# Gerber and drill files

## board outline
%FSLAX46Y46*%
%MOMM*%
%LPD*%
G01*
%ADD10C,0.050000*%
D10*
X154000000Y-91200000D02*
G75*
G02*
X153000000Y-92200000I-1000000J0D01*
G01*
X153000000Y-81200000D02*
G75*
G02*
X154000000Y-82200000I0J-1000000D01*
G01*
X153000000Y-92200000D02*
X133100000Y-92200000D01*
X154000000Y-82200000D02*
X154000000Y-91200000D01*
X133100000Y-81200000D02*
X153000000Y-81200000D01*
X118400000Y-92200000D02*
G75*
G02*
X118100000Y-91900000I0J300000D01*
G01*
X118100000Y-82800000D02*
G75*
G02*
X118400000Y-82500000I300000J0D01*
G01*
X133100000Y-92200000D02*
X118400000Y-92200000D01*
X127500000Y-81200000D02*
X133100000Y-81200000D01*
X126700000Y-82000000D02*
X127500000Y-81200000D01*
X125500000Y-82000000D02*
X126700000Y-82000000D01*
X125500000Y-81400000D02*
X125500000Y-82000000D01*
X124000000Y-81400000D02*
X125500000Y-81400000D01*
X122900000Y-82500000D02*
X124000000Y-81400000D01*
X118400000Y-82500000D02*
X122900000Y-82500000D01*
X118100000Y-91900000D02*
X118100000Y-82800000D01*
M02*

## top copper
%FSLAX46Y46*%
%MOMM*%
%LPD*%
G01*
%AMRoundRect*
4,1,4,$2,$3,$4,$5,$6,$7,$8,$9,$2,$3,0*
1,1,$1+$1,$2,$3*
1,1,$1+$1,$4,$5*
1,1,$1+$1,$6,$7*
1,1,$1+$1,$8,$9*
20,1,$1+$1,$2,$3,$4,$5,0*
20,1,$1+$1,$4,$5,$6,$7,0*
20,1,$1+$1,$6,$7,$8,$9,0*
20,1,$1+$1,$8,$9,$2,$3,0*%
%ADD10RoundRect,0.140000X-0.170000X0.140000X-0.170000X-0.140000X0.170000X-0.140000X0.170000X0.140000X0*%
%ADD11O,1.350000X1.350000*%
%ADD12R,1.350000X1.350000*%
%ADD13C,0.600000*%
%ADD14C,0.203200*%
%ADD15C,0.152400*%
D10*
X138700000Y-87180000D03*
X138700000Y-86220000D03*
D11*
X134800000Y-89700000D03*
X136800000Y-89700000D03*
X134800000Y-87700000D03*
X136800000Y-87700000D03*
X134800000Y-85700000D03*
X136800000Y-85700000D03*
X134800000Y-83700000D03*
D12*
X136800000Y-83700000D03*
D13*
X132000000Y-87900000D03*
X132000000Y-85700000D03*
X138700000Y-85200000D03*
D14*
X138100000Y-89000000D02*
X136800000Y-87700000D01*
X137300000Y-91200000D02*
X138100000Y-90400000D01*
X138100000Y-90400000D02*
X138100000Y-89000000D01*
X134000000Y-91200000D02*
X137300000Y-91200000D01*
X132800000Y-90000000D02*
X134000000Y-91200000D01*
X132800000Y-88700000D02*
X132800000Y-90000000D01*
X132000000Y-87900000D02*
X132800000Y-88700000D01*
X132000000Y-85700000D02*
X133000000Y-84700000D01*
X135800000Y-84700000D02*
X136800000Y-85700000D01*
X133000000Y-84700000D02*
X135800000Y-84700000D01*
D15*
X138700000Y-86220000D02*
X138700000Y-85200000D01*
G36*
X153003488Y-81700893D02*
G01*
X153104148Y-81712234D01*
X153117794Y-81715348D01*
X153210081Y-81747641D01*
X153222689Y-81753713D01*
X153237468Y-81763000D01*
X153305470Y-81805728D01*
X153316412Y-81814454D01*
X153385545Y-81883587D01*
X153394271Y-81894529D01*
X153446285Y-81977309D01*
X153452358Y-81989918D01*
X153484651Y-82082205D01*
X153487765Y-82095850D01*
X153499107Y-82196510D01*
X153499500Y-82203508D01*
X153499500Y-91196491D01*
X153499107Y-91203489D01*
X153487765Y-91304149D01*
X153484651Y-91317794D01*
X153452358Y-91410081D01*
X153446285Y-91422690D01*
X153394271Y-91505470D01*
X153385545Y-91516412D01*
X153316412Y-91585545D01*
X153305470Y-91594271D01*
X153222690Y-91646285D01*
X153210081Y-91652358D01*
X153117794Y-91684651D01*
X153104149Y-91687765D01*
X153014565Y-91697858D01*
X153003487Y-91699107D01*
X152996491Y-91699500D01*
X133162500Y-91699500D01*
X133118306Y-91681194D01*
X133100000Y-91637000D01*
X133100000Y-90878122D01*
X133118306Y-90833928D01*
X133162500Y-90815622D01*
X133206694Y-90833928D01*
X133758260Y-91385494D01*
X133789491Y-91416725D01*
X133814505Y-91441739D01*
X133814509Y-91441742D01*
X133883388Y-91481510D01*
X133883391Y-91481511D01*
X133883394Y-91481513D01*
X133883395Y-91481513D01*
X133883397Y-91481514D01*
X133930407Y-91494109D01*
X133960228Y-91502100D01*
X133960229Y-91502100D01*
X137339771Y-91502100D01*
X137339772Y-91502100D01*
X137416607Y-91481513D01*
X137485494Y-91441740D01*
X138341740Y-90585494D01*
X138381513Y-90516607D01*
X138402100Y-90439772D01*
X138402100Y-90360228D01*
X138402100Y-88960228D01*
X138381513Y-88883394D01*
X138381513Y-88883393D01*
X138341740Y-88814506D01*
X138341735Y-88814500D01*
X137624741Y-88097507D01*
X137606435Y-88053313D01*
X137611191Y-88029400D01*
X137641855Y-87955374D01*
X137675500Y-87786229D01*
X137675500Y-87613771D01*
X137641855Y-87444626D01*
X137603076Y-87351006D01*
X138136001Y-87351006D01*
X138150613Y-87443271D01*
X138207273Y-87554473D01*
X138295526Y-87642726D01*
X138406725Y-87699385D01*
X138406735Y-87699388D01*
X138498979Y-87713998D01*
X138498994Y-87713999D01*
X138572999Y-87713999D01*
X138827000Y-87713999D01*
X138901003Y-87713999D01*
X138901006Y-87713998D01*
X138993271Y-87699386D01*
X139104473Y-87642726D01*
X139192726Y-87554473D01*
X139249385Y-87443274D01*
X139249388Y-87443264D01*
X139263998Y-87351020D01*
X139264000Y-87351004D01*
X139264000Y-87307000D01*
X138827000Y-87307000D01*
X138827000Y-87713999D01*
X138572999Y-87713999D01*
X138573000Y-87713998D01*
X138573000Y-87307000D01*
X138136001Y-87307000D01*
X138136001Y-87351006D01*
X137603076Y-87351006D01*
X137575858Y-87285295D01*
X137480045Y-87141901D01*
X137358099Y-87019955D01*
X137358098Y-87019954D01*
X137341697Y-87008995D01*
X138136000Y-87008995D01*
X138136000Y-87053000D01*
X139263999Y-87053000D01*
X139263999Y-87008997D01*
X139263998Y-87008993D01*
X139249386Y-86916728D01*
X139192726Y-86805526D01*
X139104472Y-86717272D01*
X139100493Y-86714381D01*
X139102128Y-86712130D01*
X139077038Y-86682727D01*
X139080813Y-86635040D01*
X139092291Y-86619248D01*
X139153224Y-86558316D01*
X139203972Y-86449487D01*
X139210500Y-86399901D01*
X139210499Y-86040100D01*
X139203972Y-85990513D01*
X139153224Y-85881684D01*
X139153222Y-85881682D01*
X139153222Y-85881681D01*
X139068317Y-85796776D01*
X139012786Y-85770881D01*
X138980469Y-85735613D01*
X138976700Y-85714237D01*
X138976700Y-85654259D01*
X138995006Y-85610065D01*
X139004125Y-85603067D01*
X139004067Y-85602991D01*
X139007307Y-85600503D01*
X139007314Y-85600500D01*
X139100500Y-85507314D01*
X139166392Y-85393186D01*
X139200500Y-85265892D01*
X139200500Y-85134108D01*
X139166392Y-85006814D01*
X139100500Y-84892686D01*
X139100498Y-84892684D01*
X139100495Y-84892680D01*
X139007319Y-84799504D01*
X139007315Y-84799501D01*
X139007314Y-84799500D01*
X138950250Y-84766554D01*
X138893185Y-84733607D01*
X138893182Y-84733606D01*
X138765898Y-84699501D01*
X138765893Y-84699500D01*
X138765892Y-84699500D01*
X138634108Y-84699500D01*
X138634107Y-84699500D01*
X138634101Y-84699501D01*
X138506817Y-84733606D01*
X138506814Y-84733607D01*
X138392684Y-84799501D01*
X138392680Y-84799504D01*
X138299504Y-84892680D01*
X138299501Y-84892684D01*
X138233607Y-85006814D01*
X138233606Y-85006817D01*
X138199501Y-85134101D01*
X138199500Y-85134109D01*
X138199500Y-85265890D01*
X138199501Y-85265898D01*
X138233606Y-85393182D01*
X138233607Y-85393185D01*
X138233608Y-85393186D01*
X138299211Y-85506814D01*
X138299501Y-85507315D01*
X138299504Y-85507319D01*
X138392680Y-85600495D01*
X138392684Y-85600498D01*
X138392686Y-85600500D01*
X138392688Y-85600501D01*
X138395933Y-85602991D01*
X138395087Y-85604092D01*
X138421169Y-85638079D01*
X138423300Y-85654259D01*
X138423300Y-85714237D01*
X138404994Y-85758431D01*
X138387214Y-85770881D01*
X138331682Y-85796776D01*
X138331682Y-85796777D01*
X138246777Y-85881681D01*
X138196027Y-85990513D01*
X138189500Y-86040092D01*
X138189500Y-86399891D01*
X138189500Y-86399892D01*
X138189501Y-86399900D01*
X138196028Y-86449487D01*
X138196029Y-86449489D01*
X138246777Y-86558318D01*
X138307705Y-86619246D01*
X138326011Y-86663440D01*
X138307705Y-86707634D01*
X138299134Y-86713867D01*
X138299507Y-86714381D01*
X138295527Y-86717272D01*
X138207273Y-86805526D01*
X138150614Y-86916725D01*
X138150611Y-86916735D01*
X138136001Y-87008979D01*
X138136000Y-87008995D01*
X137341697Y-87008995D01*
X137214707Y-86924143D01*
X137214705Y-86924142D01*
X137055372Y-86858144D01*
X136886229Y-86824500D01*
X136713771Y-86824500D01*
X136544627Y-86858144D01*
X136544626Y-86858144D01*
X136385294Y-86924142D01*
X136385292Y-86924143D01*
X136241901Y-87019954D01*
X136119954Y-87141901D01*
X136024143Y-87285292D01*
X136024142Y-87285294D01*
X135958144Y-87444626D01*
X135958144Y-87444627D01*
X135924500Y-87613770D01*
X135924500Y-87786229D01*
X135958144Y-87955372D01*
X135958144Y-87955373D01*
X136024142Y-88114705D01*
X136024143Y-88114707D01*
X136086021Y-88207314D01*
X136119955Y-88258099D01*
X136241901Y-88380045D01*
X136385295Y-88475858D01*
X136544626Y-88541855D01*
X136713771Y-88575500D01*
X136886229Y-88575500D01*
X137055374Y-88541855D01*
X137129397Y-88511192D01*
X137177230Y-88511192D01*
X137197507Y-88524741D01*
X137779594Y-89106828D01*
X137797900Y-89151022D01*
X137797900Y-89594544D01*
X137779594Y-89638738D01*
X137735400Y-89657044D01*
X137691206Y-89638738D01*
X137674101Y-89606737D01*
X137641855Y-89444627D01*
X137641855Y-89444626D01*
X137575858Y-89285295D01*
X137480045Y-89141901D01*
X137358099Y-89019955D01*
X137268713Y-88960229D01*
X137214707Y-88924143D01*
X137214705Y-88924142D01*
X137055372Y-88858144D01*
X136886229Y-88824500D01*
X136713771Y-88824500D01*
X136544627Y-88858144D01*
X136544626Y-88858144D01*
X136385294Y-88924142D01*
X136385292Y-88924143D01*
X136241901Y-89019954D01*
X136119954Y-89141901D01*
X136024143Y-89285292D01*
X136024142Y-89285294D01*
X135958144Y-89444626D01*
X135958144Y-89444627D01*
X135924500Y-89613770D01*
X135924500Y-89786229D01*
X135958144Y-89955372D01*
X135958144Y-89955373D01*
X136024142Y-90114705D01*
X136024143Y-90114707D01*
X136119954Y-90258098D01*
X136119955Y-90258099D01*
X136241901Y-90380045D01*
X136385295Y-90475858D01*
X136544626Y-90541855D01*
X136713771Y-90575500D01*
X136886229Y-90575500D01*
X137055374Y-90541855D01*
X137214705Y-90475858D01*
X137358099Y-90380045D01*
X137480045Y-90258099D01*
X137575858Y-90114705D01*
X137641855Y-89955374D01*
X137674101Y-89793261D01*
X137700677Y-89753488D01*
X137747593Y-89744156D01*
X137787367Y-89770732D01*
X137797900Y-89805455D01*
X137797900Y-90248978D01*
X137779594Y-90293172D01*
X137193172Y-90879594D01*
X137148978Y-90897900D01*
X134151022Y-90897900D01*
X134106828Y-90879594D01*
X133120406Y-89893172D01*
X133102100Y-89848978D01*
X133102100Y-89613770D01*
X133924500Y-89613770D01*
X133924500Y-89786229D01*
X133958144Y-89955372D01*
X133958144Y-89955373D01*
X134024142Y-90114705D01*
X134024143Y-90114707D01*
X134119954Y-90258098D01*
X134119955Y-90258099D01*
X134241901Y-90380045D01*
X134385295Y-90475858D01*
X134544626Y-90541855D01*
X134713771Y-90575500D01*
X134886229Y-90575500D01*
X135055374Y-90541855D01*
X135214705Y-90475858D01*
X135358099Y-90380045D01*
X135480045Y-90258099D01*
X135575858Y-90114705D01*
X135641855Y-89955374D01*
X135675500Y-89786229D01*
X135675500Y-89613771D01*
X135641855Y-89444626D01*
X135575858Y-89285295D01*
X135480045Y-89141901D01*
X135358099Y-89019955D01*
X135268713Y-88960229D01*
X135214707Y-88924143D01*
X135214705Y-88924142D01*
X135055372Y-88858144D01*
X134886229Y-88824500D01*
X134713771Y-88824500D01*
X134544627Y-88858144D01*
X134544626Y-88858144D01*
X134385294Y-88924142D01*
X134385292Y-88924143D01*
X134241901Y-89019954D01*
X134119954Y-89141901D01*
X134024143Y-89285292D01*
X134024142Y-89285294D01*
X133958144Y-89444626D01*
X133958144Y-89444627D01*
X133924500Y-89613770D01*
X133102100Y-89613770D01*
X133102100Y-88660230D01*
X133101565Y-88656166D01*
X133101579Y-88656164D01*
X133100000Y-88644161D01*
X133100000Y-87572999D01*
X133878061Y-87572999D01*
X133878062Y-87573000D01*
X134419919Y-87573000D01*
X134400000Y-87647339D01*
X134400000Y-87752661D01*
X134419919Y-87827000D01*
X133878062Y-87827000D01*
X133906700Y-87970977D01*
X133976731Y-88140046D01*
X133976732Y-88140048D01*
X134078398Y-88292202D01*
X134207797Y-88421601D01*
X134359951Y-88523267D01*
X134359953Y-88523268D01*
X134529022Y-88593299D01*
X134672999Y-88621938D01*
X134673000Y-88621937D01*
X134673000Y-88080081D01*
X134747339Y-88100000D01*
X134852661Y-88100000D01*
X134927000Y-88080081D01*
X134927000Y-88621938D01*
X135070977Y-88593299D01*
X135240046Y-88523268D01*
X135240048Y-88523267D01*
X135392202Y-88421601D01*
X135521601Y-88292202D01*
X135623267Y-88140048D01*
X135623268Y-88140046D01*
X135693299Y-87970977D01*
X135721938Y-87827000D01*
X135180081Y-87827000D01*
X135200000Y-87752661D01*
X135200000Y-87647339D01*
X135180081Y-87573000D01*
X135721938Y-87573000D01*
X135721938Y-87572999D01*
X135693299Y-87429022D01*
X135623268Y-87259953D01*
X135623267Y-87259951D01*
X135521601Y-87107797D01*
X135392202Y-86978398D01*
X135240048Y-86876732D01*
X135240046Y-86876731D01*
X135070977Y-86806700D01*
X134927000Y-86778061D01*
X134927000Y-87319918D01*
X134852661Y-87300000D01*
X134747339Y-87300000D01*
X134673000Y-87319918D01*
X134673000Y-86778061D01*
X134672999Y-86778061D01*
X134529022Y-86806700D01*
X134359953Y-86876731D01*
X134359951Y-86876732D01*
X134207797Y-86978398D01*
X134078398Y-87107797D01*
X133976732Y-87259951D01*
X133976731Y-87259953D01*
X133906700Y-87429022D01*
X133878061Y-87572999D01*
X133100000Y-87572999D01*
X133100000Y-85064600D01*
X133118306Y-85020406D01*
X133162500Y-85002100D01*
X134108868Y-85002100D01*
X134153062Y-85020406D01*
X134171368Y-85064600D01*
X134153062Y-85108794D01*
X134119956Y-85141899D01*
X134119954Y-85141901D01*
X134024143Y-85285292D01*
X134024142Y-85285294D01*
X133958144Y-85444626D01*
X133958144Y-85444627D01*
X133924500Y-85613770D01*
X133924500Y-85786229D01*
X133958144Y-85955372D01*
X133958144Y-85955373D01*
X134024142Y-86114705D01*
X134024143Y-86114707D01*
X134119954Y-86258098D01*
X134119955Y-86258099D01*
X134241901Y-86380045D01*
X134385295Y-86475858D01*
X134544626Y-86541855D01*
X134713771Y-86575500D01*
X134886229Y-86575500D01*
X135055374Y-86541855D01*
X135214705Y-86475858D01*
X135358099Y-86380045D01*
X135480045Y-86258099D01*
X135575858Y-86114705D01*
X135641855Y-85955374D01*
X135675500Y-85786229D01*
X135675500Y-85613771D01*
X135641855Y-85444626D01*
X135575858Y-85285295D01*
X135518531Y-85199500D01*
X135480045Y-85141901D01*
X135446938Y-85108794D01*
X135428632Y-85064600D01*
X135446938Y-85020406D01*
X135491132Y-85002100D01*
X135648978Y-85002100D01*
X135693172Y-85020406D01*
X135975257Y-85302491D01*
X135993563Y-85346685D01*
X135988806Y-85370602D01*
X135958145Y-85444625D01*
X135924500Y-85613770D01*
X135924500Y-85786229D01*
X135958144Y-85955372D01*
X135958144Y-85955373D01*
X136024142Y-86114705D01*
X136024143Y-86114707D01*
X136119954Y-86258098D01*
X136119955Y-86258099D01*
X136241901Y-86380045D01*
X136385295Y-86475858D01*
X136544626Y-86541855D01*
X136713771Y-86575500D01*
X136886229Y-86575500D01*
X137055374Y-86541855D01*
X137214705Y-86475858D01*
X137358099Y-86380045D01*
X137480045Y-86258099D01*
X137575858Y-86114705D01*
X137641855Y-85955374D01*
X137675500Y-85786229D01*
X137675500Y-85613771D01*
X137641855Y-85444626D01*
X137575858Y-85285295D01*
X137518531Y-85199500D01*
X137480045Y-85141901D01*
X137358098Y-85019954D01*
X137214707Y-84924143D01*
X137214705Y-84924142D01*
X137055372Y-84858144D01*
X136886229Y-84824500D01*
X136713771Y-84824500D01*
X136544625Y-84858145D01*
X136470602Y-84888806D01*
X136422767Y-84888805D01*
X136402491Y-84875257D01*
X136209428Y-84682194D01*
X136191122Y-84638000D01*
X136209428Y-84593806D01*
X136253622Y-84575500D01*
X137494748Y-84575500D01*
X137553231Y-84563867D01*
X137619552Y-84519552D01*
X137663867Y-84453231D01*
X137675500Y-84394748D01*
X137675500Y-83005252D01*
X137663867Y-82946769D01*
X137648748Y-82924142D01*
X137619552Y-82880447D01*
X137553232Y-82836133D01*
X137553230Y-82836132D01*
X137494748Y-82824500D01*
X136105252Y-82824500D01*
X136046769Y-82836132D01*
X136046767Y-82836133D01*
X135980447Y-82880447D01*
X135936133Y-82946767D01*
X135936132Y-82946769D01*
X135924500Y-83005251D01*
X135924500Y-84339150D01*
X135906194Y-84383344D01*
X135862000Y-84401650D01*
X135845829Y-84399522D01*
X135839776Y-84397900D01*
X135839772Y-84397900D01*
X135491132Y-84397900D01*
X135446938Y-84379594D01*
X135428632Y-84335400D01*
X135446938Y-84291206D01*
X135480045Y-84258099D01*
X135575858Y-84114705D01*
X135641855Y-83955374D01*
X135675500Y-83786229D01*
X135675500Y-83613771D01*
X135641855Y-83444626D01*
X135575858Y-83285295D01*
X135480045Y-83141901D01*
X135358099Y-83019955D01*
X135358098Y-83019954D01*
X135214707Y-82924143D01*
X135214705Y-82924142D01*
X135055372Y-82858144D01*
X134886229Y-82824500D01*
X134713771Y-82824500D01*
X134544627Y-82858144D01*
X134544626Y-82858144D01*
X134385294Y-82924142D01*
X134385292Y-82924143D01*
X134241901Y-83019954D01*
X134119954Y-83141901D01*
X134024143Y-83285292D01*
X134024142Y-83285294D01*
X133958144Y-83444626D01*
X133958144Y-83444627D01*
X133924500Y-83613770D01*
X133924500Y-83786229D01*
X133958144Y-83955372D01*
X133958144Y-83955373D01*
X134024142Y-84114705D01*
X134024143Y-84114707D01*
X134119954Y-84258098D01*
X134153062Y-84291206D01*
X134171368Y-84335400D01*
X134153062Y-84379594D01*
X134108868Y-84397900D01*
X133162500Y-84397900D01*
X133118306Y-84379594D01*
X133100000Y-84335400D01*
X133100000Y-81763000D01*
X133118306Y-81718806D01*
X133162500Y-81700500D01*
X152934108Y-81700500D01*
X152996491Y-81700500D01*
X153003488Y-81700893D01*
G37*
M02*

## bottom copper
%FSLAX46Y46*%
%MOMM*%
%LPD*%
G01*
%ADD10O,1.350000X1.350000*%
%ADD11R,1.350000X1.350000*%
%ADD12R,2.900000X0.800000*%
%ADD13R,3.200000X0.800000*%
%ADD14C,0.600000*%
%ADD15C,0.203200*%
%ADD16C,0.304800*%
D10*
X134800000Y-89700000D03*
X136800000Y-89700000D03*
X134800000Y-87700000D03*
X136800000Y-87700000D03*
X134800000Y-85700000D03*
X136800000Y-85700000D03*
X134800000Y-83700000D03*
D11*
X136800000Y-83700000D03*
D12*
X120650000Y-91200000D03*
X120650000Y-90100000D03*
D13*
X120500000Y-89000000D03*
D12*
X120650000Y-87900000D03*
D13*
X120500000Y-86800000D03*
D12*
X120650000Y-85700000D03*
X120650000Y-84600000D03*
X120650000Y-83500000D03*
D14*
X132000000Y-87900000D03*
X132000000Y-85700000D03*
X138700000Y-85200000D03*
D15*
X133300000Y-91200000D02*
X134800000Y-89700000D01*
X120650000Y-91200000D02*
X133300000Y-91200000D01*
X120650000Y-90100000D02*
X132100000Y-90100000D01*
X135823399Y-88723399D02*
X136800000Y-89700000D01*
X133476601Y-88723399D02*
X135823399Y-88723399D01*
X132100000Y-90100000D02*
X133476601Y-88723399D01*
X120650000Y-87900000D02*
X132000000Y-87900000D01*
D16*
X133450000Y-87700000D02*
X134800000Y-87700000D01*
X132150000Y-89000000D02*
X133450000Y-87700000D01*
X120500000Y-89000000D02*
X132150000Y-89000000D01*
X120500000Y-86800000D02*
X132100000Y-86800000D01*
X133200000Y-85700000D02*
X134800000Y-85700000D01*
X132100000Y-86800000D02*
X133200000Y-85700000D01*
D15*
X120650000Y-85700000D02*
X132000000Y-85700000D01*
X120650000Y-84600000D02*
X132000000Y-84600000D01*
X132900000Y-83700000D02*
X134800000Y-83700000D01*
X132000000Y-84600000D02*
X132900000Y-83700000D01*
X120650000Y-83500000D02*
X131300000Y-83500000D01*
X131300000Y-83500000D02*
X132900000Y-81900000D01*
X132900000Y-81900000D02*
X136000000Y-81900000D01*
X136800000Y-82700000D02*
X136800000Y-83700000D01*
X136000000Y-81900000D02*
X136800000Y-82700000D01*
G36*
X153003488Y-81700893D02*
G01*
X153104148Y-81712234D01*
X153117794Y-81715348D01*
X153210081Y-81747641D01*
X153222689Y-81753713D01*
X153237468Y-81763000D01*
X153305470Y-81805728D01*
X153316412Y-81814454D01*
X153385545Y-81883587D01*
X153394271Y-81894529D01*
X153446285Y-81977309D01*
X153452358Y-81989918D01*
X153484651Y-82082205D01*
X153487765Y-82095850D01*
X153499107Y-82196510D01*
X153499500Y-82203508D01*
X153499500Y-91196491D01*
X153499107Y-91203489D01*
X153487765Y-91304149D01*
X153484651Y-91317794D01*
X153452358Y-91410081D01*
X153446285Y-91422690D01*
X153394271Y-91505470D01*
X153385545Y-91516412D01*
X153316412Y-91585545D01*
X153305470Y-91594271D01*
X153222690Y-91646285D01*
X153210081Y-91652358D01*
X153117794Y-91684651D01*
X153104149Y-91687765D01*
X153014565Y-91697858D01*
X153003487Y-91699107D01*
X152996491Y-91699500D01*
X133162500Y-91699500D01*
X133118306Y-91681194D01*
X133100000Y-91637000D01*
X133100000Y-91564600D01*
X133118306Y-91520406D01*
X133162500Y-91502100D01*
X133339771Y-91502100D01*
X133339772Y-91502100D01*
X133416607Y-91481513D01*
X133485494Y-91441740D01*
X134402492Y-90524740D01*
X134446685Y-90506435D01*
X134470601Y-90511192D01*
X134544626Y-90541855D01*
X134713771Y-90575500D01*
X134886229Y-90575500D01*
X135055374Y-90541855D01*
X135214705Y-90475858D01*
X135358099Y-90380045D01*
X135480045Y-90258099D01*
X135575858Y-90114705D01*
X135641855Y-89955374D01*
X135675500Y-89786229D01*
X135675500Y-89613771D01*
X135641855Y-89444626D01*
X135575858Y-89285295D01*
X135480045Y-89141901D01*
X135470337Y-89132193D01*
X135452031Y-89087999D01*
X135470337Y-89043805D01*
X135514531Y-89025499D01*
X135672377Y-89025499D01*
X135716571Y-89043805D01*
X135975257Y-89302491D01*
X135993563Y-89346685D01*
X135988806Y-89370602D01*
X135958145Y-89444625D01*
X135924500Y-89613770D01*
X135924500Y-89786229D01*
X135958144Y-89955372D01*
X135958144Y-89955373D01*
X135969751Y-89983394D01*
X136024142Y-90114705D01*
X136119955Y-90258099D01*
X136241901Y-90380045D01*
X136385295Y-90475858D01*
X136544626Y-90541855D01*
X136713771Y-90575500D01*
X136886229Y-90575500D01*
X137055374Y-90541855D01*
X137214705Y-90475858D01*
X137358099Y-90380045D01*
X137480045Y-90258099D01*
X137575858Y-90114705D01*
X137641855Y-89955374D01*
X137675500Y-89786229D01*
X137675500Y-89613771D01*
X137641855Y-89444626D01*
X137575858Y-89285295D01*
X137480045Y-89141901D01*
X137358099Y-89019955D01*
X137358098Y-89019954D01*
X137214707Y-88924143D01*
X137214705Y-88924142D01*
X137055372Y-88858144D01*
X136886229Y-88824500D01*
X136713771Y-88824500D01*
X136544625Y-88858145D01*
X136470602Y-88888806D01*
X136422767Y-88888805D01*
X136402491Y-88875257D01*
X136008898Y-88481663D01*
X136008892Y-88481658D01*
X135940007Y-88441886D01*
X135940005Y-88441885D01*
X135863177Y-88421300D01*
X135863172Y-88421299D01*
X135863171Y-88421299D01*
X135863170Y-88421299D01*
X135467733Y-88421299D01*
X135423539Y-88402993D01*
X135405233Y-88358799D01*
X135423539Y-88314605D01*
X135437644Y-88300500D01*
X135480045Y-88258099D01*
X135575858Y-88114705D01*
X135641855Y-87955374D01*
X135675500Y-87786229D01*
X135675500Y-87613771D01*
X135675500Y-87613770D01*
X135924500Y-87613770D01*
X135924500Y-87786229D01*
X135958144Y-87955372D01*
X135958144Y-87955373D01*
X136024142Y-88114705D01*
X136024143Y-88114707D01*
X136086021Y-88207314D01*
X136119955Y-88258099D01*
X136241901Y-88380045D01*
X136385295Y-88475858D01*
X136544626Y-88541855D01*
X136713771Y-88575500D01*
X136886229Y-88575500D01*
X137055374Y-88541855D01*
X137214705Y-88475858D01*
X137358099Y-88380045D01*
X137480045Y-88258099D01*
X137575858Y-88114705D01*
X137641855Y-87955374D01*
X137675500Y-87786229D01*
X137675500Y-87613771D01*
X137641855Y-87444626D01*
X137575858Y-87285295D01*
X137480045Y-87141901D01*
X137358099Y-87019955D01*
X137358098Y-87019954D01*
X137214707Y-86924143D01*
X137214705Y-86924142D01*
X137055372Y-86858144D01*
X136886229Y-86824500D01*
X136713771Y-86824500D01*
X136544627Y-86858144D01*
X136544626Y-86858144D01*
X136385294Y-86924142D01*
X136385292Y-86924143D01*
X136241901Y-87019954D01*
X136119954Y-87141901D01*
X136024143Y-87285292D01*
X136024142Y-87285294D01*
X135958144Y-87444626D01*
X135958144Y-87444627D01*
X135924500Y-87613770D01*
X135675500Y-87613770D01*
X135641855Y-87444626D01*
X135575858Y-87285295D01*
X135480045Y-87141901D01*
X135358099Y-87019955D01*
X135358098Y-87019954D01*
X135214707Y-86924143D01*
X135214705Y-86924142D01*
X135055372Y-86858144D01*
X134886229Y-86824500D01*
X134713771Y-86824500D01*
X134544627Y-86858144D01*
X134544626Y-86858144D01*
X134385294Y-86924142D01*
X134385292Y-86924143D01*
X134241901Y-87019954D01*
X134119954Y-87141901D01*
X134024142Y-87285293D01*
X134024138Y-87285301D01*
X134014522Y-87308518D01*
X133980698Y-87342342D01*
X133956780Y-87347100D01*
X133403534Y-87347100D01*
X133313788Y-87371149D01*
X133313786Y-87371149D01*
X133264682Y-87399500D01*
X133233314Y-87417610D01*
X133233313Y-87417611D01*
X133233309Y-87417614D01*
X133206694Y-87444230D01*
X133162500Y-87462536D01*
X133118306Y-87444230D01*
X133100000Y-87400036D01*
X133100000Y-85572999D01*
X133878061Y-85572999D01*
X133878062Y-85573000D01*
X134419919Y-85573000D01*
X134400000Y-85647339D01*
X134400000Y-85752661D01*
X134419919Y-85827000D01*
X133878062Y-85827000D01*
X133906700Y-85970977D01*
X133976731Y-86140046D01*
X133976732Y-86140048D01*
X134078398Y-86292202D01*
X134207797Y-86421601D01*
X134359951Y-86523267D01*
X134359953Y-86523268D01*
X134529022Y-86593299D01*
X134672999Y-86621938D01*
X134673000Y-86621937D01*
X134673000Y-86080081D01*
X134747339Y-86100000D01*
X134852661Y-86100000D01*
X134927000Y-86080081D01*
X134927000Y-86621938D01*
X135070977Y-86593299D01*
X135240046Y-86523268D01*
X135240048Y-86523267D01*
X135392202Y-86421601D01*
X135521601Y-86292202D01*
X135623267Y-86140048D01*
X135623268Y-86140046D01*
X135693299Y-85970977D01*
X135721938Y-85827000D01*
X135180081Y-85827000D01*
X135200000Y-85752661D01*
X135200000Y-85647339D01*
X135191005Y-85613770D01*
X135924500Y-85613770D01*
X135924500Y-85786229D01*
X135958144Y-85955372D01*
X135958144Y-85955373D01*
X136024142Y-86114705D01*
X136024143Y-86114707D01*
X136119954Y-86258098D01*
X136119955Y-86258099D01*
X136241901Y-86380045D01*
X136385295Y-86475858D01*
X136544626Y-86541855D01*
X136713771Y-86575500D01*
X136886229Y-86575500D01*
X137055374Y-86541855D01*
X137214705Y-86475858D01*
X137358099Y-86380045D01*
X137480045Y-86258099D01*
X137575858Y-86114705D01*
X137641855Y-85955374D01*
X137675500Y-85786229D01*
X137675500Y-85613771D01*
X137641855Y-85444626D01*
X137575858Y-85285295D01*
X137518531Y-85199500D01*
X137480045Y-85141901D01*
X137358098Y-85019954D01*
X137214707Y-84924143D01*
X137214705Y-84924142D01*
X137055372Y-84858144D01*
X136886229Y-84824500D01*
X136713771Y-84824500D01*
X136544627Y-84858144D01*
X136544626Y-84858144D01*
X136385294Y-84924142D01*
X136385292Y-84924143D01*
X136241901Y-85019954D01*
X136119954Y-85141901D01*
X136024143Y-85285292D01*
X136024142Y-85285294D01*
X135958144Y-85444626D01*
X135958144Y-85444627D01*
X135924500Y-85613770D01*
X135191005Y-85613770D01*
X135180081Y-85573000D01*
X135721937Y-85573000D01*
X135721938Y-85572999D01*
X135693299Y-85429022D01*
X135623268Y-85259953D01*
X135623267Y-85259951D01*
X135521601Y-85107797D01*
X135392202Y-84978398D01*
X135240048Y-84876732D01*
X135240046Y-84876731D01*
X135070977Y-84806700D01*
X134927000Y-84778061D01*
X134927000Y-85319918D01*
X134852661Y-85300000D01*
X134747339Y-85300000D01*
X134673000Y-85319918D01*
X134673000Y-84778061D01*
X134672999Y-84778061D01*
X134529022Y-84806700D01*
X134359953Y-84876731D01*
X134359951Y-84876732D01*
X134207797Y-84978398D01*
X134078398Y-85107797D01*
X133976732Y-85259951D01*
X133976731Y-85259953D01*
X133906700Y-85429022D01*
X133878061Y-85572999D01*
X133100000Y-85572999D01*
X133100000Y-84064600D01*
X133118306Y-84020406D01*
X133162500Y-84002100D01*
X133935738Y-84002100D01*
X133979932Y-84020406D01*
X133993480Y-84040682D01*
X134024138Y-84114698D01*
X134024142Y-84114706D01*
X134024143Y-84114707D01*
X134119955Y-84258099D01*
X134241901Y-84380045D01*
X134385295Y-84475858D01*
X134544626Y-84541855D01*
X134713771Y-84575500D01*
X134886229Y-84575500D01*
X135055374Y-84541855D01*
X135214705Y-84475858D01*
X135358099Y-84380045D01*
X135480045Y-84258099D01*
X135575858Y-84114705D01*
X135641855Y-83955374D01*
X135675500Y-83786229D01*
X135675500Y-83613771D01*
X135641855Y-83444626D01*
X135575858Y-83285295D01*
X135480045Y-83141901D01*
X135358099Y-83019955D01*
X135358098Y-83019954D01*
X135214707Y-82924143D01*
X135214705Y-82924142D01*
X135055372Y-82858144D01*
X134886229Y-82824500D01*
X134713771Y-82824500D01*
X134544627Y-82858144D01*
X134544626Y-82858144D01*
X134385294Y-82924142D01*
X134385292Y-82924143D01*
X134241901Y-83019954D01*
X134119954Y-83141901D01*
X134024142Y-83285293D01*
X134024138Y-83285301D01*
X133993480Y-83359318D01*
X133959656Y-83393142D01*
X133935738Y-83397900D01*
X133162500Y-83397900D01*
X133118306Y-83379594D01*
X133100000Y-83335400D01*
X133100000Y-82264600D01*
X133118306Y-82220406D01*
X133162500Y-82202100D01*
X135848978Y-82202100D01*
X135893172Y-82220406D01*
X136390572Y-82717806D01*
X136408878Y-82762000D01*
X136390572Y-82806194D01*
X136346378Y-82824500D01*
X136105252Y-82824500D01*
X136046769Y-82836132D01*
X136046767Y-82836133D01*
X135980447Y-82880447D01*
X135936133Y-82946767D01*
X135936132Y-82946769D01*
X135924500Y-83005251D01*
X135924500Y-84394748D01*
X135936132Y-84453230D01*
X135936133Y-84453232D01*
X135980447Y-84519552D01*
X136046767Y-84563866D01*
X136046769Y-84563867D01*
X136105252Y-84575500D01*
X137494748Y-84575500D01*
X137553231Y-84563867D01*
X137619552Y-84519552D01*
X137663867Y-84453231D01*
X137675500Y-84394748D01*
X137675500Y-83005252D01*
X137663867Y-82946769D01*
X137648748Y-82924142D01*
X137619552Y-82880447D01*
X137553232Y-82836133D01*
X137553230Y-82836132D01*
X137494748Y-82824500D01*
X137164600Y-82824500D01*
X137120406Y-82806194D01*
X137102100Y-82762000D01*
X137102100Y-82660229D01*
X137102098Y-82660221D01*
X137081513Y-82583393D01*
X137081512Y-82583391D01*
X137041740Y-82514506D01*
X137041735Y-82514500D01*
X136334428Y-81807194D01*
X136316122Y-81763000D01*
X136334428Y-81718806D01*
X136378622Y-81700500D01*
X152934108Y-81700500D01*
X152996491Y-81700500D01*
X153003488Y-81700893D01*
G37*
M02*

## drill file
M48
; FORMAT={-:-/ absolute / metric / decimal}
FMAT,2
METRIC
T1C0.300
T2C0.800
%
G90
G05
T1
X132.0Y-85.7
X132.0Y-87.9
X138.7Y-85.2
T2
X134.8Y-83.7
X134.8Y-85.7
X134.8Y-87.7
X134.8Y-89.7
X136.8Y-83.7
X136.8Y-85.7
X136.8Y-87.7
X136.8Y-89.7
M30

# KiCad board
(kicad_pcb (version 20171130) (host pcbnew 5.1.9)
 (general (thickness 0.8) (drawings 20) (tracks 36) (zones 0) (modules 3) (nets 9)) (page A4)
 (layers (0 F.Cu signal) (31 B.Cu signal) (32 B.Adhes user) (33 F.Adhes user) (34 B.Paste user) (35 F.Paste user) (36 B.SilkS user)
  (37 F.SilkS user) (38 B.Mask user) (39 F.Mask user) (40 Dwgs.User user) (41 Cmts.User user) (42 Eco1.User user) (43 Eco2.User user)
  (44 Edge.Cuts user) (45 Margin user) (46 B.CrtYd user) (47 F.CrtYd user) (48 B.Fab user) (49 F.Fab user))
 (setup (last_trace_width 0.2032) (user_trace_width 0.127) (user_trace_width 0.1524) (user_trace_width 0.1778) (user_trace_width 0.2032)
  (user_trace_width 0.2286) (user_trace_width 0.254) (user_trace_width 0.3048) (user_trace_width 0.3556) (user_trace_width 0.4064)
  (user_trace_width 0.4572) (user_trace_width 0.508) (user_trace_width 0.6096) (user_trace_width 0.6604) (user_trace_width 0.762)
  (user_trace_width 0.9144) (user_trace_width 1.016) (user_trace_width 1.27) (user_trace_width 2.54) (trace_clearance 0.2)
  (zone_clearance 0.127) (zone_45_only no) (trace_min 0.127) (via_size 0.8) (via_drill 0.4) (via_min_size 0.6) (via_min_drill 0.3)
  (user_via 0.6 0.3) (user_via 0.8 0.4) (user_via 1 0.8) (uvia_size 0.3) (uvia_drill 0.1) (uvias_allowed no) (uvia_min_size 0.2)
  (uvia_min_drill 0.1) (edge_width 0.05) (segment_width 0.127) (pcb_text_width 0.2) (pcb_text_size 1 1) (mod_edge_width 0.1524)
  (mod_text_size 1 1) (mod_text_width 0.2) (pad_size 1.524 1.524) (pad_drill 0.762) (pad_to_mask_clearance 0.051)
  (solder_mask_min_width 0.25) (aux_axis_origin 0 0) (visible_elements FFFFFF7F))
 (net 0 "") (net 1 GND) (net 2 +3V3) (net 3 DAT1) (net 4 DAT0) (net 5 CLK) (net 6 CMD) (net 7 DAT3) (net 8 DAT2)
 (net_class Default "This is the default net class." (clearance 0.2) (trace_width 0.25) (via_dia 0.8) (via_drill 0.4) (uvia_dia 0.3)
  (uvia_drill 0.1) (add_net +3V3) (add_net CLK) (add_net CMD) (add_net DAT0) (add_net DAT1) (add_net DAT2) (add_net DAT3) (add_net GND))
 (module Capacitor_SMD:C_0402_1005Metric (layer F.Cu) (at 138.7 86.7 270)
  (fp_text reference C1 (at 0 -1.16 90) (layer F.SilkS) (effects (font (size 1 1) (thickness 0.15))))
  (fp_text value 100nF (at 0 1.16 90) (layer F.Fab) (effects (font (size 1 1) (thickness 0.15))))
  (pad 2 smd roundrect (at 0.48 0 270) (size 0.56 0.62) (layers F.Cu F.Paste F.Mask) (roundrect_rratio 0.25) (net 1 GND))
  (pad 1 smd roundrect (at -0.48 0 270) (size 0.56 0.62) (layers F.Cu F.Paste F.Mask) (roundrect_rratio 0.25) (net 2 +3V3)))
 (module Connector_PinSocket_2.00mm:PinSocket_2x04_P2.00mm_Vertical (layer F.Cu) (at 136.8 83.7)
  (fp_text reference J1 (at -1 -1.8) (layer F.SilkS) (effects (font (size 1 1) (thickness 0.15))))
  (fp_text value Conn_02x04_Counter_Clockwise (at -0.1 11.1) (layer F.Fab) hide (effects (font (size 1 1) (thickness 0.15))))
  (pad 8 thru_hole oval (at -2 6) (size 1.35 1.35) (drill 0.8) (layers *.Cu *.Mask) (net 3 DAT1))
  (pad 7 thru_hole oval (at 0 6) (size 1.35 1.35) (drill 0.8) (layers *.Cu *.Mask) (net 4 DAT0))
  (pad 6 thru_hole oval (at -2 4) (size 1.35 1.35) (drill 0.8) (layers *.Cu *.Mask) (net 1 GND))
  (pad 5 thru_hole oval (at 0 4) (size 1.35 1.35) (drill 0.8) (layers *.Cu *.Mask) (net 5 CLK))
  (pad 4 thru_hole oval (at -2 2) (size 1.35 1.35) (drill 0.8) (layers *.Cu *.Mask) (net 2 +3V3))
  (pad 3 thru_hole oval (at 0 2) (size 1.35 1.35) (drill 0.8) (layers *.Cu *.Mask) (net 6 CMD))
  (pad 2 thru_hole oval (at -2 0) (size 1.35 1.35) (drill 0.8) (layers *.Cu *.Mask) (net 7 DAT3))
  (pad 1 thru_hole rect (at 0 0) (size 1.35 1.35) (drill 0.8) (layers *.Cu *.Mask) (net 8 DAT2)))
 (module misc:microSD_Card (layer F.Cu) (at 125.6 87.3)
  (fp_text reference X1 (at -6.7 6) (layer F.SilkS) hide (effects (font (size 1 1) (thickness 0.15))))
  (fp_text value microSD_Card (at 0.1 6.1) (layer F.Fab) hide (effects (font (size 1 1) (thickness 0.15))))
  (pad 8 smd rect (at -4.95 3.9 270) (size 0.8 2.9) (layers B.Cu B.Paste B.Mask) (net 3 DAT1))
  (pad 7 smd rect (at -4.95 2.8 270) (size 0.8 2.9) (layers B.Cu B.Paste B.Mask) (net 4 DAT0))
  (pad 6 smd rect (at -5.1 1.7 270) (size 0.8 3.2) (layers B.Cu B.Paste B.Mask) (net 1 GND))
  (pad 5 smd rect (at -4.95 0.6 270) (size 0.8 2.9) (layers B.Cu B.Paste B.Mask) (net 5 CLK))
  (pad 4 smd rect (at -5.1 -0.5 270) (size 0.8 3.2) (layers B.Cu B.Paste B.Mask) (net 2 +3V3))
  (pad 3 smd rect (at -4.95 -1.6 270) (size 0.8 2.9) (layers B.Cu B.Paste B.Mask) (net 6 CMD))
  (pad 2 smd rect (at -4.95 -2.7 270) (size 0.8 2.9) (layers B.Cu B.Paste B.Mask) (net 7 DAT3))
  (pad 1 smd rect (at -4.95 -3.8 270) (size 0.8 2.9) (layers B.Cu B.Paste B.Mask) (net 8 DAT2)))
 (gr_arc (start 153 91.2) (end 153 92.2) (angle -90) (layer Edge.Cuts) (width 0.05))
 (gr_arc (start 153 82.2) (end 154 82.2) (angle -90) (layer Edge.Cuts) (width 0.05))
 (gr_line (start 153 92.2) (end 133.1 92.2) (layer Edge.Cuts) (width 0.05))
 (gr_line (start 154 82.2) (end 154 91.2) (layer Edge.Cuts) (width 0.05))
 (gr_line (start 133.1 81.2) (end 153 81.2) (layer Edge.Cuts) (width 0.05))
 (gr_arc (start 118.4 91.9) (end 118.1 91.9) (angle -90) (layer Edge.Cuts) (width 0.05))
 (gr_arc (start 118.4 82.8) (end 118.4 82.5) (angle -90) (layer Edge.Cuts) (width 0.05))
 (gr_line (start 133.1 92.2) (end 118.4 92.2) (layer Edge.Cuts) (width 0.05))
 (gr_line (start 127.5 81.2) (end 133.1 81.2) (layer Edge.Cuts) (width 0.05))
 (gr_line (start 126.7 82) (end 127.5 81.2) (layer Edge.Cuts) (width 0.05))
 (gr_line (start 125.5 82) (end 126.7 82) (layer Edge.Cuts) (width 0.05))
 (gr_line (start 125.5 81.4) (end 125.5 82) (layer Edge.Cuts) (width 0.05))
 (gr_line (start 124 81.4) (end 125.5 81.4) (layer Edge.Cuts) (width 0.05))
 (gr_line (start 122.9 82.5) (end 124 81.4) (layer Edge.Cuts) (width 0.05))
 (gr_line (start 118.4 82.5) (end 122.9 82.5) (layer Edge.Cuts) (width 0.05))
 (gr_line (start 118.1 91.9) (end 118.1 82.8) (layer Edge.Cuts) (width 0.05))
 (segment (start 133.3 91.2) (end 134.8 89.7) (width 0.2032) (layer B.Cu) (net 3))
 (segment (start 120.65 91.2) (end 133.3 91.2) (width 0.2032) (layer B.Cu) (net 3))
 (segment (start 120.65 90.1) (end 132.1 90.1) (width 0.2032) (layer B.Cu) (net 4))
 (segment (start 135.823399 88.723399) (end 136.8 89.7) (width 0.2032) (layer B.Cu) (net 4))
 (segment (start 133.476601 88.723399) (end 135.823399 88.723399) (width 0.2032) (layer B.Cu) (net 4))
 (segment (start 132.1 90.1) (end 133.476601 88.723399) (width 0.2032) (layer B.Cu) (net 4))
 (via (at 132 87.9) (size 0.6) (drill 0.3) (layers F.Cu B.Cu) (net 5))
 (segment (start 120.65 87.9) (end 132 87.9) (width 0.2032) (layer B.Cu) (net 5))
 (segment (start 138.1 89) (end 136.8 87.7) (width 0.2032) (layer F.Cu) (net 5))
 (segment (start 137.3 91.2) (end 138.1 90.4) (width 0.2032) (layer F.Cu) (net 5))
 (segment (start 138.1 90.4) (end 138.1 89) (width 0.2032) (layer F.Cu) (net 5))
 (segment (start 134 91.2) (end 137.3 91.2) (width 0.2032) (layer F.Cu) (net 5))
 (segment (start 132.8 90) (end 134 91.2) (width 0.2032) (layer F.Cu) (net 5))
 (segment (start 132.8 88.7) (end 132.8 90) (width 0.2032) (layer F.Cu) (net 5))
 (segment (start 132 87.9) (end 132.8 88.7) (width 0.2032) (layer F.Cu) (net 5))
 (segment (start 133.45 87.7) (end 134.8 87.7) (width 0.3048) (layer B.Cu) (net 1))
 (segment (start 132.15 89) (end 133.45 87.7) (width 0.3048) (layer B.Cu) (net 1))
 (segment (start 120.5 89) (end 132.15 89) (width 0.3048) (layer B.Cu) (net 1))
 (segment (start 120.5 86.8) (end 132.1 86.8) (width 0.3048) (layer B.Cu) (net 2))
 (segment (start 133.2 85.7) (end 134.8 85.7) (width 0.3048) (layer B.Cu) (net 2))
 (segment (start 132.1 86.8) (end 133.2 85.7) (width 0.3048) (layer B.Cu) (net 2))
 (segment (start 120.65 85.7) (end 132 85.7) (width 0.2032) (layer B.Cu) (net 6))
 (via (at 132 85.7) (size 0.6) (drill 0.3) (layers F.Cu B.Cu) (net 6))
 (segment (start 132 85.7) (end 133 84.7) (width 0.2032) (layer F.Cu) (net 6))
 (segment (start 135.8 84.7) (end 136.8 85.7) (width 0.2032) (layer F.Cu) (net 6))
 (segment (start 133 84.7) (end 135.8 84.7) (width 0.2032) (layer F.Cu) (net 6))
 (segment (start 120.65 84.6) (end 132 84.6) (width 0.2032) (layer B.Cu) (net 7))
 (segment (start 132.9 83.7) (end 134.8 83.7) (width 0.2032) (layer B.Cu) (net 7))
 (segment (start 132 84.6) (end 132.9 83.7) (width 0.2032) (layer B.Cu) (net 7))
 (segment (start 120.65 83.5) (end 131.3 83.5) (width 0.2032) (layer B.Cu) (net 8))
 (segment (start 131.3 83.5) (end 132.9 81.9) (width 0.2032) (layer B.Cu) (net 8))
 (segment (start 132.9 81.9) (end 136 81.9) (width 0.2032) (layer B.Cu) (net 8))
 (segment (start 136.8 82.7) (end 136.8 83.7) (width 0.2032) (layer B.Cu) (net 8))
 (segment (start 136 81.9) (end 136.8 82.7) (width 0.2032) (layer B.Cu) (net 8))
 (via (at 138.7 85.2) (size 0.6) (drill 0.3) (layers F.Cu B.Cu) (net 2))
 (segment (start 138.7 86.22) (end 138.7 85.2) (width 0.1524) (layer F.Cu) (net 2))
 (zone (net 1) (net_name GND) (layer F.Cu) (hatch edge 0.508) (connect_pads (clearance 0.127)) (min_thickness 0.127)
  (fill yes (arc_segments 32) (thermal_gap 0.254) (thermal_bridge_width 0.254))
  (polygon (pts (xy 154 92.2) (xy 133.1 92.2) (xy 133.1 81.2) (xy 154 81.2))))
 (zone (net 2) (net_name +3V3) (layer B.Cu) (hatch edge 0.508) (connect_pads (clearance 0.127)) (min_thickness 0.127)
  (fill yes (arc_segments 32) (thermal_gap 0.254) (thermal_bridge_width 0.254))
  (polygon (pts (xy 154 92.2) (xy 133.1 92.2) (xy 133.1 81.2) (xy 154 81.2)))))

